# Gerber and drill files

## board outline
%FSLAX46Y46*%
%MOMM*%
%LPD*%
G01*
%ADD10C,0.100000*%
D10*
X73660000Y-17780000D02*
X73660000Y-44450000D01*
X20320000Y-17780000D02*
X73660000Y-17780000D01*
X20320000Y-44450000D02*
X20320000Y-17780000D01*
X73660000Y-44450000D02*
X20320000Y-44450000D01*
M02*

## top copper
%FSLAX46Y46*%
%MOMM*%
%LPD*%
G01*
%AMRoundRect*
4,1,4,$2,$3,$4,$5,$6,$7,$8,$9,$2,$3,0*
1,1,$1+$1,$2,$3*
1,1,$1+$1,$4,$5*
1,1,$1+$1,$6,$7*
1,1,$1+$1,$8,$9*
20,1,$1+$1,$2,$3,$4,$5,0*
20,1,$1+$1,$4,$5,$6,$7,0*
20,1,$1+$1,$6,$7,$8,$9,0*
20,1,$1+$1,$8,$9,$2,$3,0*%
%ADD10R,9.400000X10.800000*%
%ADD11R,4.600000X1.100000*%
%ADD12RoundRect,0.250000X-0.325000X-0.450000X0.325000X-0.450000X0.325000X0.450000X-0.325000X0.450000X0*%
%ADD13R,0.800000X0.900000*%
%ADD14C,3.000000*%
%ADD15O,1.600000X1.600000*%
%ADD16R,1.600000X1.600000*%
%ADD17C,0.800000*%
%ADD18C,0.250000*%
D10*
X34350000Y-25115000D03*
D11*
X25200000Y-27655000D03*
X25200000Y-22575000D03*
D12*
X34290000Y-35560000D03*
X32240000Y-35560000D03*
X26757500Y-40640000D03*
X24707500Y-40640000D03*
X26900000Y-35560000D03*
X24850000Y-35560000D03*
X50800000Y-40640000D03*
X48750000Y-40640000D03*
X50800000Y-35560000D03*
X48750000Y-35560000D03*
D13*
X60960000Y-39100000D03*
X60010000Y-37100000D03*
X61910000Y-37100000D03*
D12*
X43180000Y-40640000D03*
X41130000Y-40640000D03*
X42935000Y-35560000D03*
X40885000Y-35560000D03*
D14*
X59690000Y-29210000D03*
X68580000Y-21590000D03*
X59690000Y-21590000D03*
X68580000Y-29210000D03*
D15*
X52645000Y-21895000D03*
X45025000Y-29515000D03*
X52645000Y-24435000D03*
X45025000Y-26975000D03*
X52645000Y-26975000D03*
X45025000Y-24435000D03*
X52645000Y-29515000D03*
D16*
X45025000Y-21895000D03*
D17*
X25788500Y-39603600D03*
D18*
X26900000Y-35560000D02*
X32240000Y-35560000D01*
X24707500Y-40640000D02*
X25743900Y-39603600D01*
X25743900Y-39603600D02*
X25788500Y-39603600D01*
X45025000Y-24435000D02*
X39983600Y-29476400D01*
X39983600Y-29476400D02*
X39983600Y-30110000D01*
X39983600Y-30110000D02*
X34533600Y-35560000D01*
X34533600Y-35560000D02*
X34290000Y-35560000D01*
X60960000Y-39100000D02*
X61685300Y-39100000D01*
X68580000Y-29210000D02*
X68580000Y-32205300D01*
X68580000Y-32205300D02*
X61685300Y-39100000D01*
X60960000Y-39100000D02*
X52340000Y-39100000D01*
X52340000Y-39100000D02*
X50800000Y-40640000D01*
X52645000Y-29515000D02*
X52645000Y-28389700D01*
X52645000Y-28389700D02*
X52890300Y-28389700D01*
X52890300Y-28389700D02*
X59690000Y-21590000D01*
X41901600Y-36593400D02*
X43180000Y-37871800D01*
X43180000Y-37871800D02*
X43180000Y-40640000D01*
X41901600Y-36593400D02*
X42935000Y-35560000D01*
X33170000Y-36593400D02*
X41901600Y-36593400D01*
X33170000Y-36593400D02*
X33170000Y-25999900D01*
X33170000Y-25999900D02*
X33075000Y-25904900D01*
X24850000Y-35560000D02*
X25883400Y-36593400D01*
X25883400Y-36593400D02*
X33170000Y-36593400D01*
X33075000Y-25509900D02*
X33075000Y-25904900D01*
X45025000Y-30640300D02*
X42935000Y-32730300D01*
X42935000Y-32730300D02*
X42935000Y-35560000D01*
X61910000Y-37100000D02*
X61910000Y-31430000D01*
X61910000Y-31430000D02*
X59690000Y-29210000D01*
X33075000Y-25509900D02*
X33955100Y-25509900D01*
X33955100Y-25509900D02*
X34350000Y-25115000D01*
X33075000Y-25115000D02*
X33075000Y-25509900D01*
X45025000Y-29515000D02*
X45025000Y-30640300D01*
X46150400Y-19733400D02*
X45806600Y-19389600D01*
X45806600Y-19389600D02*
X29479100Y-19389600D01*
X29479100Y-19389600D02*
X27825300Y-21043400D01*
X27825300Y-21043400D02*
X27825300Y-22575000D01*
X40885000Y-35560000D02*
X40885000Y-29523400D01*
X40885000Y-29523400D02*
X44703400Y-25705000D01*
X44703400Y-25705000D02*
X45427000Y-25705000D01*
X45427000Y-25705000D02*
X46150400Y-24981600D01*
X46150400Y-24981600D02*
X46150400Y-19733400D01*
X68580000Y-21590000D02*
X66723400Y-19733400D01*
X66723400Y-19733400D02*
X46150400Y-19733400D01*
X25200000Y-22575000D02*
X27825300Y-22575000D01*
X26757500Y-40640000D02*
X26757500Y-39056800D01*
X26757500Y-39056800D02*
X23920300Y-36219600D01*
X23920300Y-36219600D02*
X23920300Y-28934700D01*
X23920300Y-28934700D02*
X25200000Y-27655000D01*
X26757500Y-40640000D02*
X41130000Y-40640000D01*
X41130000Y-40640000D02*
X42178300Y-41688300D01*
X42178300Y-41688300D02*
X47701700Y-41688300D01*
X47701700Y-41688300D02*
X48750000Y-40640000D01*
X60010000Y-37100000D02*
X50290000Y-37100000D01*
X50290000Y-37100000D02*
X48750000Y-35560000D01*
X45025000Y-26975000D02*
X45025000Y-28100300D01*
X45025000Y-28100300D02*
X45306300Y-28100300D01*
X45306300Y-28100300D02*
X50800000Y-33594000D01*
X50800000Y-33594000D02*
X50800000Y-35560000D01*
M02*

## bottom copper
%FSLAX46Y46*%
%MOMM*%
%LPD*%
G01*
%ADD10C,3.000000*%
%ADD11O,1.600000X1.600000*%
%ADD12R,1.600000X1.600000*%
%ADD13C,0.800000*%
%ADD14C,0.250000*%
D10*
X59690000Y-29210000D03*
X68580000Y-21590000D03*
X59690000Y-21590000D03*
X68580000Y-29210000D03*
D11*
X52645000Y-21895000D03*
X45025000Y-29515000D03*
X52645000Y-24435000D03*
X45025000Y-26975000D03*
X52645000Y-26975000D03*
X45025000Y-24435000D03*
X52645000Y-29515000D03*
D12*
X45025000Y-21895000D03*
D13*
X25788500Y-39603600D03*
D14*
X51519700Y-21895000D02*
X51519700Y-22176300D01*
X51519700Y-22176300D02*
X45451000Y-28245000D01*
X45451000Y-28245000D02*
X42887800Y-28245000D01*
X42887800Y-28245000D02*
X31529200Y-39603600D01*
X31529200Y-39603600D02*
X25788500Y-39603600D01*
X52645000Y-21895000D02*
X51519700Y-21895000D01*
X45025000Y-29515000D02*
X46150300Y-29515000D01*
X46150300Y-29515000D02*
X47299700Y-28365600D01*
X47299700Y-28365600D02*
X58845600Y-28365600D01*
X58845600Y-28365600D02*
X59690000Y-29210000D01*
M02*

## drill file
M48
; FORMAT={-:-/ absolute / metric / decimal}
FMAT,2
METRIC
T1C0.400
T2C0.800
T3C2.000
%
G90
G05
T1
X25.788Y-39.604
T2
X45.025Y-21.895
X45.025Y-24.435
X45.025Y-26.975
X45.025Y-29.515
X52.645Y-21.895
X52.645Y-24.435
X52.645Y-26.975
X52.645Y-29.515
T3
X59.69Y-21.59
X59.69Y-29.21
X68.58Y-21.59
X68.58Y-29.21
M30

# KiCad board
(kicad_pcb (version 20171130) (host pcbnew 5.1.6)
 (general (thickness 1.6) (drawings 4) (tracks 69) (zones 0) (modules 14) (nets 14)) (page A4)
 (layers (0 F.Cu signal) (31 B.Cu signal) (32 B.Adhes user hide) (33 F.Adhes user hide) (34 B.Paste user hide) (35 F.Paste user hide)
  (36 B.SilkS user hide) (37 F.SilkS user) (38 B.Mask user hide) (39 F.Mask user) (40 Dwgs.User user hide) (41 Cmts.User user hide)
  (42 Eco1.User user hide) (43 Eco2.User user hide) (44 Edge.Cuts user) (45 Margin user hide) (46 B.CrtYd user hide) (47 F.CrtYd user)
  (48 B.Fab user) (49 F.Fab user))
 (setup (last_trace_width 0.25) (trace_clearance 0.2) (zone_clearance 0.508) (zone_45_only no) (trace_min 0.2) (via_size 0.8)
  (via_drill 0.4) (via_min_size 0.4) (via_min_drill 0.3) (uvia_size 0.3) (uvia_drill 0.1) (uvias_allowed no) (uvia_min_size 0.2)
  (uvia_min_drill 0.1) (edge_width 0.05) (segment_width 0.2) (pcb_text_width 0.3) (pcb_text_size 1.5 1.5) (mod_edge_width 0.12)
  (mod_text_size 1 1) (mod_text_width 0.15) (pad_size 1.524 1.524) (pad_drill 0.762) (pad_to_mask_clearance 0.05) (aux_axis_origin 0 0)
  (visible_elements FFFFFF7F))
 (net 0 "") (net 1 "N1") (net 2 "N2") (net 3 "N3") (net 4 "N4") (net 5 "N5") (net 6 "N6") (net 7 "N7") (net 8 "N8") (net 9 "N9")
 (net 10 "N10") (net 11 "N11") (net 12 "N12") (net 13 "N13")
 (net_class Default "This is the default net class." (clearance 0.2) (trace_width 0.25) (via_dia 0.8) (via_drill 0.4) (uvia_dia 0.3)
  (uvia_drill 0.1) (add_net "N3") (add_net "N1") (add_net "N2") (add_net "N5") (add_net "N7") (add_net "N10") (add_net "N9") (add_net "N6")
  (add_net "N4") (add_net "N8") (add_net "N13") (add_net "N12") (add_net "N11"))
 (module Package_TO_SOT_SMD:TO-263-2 (layer F.Cu) (at 30.975 25.115)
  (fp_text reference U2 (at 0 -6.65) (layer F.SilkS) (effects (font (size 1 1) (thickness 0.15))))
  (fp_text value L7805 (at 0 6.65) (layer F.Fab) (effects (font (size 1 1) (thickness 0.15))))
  (pad "" smd rect (at 0.95 2.775) (size 4.55 5.25) (layers F.Paste))
  (pad "" smd rect (at 5.8 -2.775) (size 4.55 5.25) (layers F.Paste))
  (pad "" smd rect (at 0.95 -2.775) (size 4.55 5.25) (layers F.Paste))
  (pad "" smd rect (at 5.8 2.775) (size 4.55 5.25) (layers F.Paste))
  (pad 2 smd rect (at 3.375 0) (size 9.4 10.8) (layers F.Cu F.Mask) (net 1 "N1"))
  (pad 3 smd rect (at -5.775 2.54) (size 4.6 1.1) (layers F.Cu F.Paste F.Mask) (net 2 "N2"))
  (pad 1 smd rect (at -5.775 -2.54) (size 4.6 1.1) (layers F.Cu F.Paste F.Mask) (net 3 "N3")))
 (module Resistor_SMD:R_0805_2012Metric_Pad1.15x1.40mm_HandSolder (layer F.Cu) (at 33.265 35.56)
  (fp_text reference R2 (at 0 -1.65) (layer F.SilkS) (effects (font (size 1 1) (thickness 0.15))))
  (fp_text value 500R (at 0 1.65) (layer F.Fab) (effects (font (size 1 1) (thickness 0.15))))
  (pad 2 smd roundrect (at 1.025 0) (size 1.15 1.4) (layers F.Cu F.Paste F.Mask) (roundrect_rratio 0.217391) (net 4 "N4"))
  (pad 1 smd roundrect (at -1.025 0) (size 1.15 1.4) (layers F.Cu F.Paste F.Mask) (roundrect_rratio 0.217391) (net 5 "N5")))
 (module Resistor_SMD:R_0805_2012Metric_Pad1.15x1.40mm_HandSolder (layer F.Cu) (at 25.7325 40.64)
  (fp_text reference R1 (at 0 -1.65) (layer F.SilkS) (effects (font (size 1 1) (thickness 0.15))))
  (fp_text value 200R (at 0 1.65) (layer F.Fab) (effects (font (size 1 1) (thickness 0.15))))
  (pad 2 smd roundrect (at 1.025 0) (size 1.15 1.4) (layers F.Cu F.Paste F.Mask) (roundrect_rratio 0.217391) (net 2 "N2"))
  (pad 1 smd roundrect (at -1.025 0) (size 1.15 1.4) (layers F.Cu F.Paste F.Mask) (roundrect_rratio 0.217391) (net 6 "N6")))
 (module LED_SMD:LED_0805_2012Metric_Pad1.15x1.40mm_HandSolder (layer F.Cu) (at 25.875 35.56)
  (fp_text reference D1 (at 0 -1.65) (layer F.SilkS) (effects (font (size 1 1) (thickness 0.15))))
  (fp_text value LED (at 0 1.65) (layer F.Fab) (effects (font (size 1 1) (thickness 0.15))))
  (pad 2 smd roundrect (at 1.025 0) (size 1.15 1.4) (layers F.Cu F.Paste F.Mask) (roundrect_rratio 0.217391) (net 5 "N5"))
  (pad 1 smd roundrect (at -1.025 0) (size 1.15 1.4) (layers F.Cu F.Paste F.Mask) (roundrect_rratio 0.217391) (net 1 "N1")))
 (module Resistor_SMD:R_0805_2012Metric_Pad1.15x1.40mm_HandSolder (layer F.Cu) (at 49.775 40.64)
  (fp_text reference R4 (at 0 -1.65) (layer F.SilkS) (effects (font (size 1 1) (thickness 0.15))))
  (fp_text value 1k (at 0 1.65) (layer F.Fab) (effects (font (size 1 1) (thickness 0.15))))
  (pad 2 smd roundrect (at 1.025 0) (size 1.15 1.4) (layers F.Cu F.Paste F.Mask) (roundrect_rratio 0.217391) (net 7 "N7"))
  (pad 1 smd roundrect (at -1.025 0) (size 1.15 1.4) (layers F.Cu F.Paste F.Mask) (roundrect_rratio 0.217391) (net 2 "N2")))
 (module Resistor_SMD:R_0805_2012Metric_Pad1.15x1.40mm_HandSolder (layer F.Cu) (at 49.775 35.56)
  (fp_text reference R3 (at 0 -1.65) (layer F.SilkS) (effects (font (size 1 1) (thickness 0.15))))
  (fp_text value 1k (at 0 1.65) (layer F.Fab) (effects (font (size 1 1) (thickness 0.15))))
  (pad 2 smd roundrect (at 1.025 0) (size 1.15 1.4) (layers F.Cu F.Paste F.Mask) (roundrect_rratio 0.217391) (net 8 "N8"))
  (pad 1 smd roundrect (at -1.025 0) (size 1.15 1.4) (layers F.Cu F.Paste F.Mask) (roundrect_rratio 0.217391) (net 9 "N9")))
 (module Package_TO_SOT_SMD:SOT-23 (layer F.Cu) (at 60.96 38.1 270)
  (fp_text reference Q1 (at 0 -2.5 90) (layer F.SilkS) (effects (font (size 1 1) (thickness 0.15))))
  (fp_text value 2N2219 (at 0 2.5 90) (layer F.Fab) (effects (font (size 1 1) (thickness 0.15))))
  (pad 3 smd rect (at 1 0 270) (size 0.9 0.8) (layers F.Cu F.Paste F.Mask) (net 7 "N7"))
  (pad 2 smd rect (at -1 0.95 270) (size 0.9 0.8) (layers F.Cu F.Paste F.Mask) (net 9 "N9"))
  (pad 1 smd rect (at -1 -0.95 270) (size 0.9 0.8) (layers F.Cu F.Paste F.Mask) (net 1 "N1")))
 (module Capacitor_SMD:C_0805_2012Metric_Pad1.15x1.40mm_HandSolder (layer F.Cu) (at 42.155 40.64)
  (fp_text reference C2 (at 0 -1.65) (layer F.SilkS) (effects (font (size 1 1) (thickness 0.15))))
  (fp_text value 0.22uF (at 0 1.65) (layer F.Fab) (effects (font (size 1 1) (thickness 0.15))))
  (pad 2 smd roundrect (at 1.025 0) (size 1.15 1.4) (layers F.Cu F.Paste F.Mask) (roundrect_rratio 0.217391) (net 1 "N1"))
  (pad 1 smd roundrect (at -1.025 0) (size 1.15 1.4) (layers F.Cu F.Paste F.Mask) (roundrect_rratio 0.217391) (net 2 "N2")))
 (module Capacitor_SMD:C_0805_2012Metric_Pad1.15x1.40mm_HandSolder (layer F.Cu) (at 41.91 35.56)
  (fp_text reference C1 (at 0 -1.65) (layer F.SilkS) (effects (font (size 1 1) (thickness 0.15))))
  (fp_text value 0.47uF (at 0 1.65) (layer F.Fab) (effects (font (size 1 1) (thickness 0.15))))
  (pad 2 smd roundrect (at 1.025 0) (size 1.15 1.4) (layers F.Cu F.Paste F.Mask) (roundrect_rratio 0.217391) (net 1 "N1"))
  (pad 1 smd roundrect (at -1.025 0) (size 1.15 1.4) (layers F.Cu F.Paste F.Mask) (roundrect_rratio 0.217391) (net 3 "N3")))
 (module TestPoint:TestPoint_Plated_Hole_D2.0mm (layer F.Cu) (at 59.69 29.21)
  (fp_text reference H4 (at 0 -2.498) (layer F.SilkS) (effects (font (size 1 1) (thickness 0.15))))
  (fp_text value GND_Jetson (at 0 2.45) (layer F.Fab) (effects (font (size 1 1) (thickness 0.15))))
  (pad 1 thru_hole circle (at 0 0) (size 3 3) (drill 2) (layers *.Cu *.Mask) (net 1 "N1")))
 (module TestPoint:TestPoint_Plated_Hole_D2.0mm (layer F.Cu) (at 68.58 21.59)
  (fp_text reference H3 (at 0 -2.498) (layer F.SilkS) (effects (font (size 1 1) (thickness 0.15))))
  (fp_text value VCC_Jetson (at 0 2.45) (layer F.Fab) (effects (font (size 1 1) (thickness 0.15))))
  (pad 1 thru_hole circle (at 0 0) (size 3 3) (drill 2) (layers *.Cu *.Mask) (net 3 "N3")))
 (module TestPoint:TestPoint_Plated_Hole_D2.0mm (layer F.Cu) (at 59.69 21.59)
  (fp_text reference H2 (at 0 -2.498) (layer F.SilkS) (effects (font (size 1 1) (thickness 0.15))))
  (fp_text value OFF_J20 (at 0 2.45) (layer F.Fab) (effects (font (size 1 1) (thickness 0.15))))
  (pad 1 thru_hole circle (at 0 0) (size 3 3) (drill 2) (layers *.Cu *.Mask) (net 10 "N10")))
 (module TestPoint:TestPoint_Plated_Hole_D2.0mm (layer F.Cu) (at 68.58 29.21)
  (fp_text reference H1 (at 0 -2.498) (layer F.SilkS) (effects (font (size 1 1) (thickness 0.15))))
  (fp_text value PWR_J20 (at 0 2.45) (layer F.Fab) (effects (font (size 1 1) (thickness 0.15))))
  (pad 1 thru_hole circle (at 0 0) (size 3 3) (drill 2) (layers *.Cu *.Mask) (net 7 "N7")))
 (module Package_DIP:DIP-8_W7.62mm (layer F.Cu) (at 45.025 21.895)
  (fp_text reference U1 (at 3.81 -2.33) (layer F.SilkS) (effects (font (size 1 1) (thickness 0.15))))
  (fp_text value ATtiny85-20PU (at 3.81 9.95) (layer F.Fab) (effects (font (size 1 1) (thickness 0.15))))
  (pad 8 thru_hole oval (at 7.62 0) (size 1.6 1.6) (drill 0.8) (layers *.Cu *.Mask) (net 6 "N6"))
  (pad 4 thru_hole oval (at 0 7.62) (size 1.6 1.6) (drill 0.8) (layers *.Cu *.Mask) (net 1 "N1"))
  (pad 7 thru_hole oval (at 7.62 2.54) (size 1.6 1.6) (drill 0.8) (layers *.Cu *.Mask) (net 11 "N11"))
  (pad 3 thru_hole oval (at 0 5.08) (size 1.6 1.6) (drill 0.8) (layers *.Cu *.Mask) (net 8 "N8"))
  (pad 6 thru_hole oval (at 7.62 5.08) (size 1.6 1.6) (drill 0.8) (layers *.Cu *.Mask) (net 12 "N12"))
  (pad 2 thru_hole oval (at 0 2.54) (size 1.6 1.6) (drill 0.8) (layers *.Cu *.Mask) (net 4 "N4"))
  (pad 5 thru_hole oval (at 7.62 7.62) (size 1.6 1.6) (drill 0.8) (layers *.Cu *.Mask) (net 10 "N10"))
  (pad 1 thru_hole rect (at 0 0) (size 1.6 1.6) (drill 0.8) (layers *.Cu *.Mask) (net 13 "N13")))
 (gr_line (start 73.66 17.78) (end 73.66 44.45) (layer Edge.Cuts) (width 0.1))
 (gr_line (start 20.32 17.78) (end 73.66 17.78) (layer Edge.Cuts) (width 0.1))
 (gr_line (start 20.32 44.45) (end 20.32 17.78) (layer Edge.Cuts) (width 0.1))
 (gr_line (start 73.66 44.45) (end 20.32 44.45) (layer Edge.Cuts) (width 0.1))
 (segment (start 26.9 35.56) (end 32.24 35.56) (width 0.25) (layer F.Cu) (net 5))
 (segment (start 24.7075 40.64) (end 25.7439 39.6036) (width 0.25) (layer F.Cu) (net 6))
 (segment (start 25.7439 39.6036) (end 25.7885 39.6036) (width 0.25) (layer F.Cu) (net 6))
 (segment (start 51.5197 21.895) (end 51.5197 22.1763) (width 0.25) (layer B.Cu) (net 6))
 (segment (start 51.5197 22.1763) (end 45.451 28.245) (width 0.25) (layer B.Cu) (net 6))
 (segment (start 45.451 28.245) (end 42.8878 28.245) (width 0.25) (layer B.Cu) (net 6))
 (segment (start 42.8878 28.245) (end 31.5292 39.6036) (width 0.25) (layer B.Cu) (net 6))
 (segment (start 31.5292 39.6036) (end 25.7885 39.6036) (width 0.25) (layer B.Cu) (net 6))
 (segment (start 52.645 21.895) (end 51.5197 21.895) (width 0.25) (layer B.Cu) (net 6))
 (via (at 25.7885 39.6036) (size 0.8) (layers F.Cu B.Cu) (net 6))
 (segment (start 45.025 24.435) (end 39.9836 29.4764) (width 0.25) (layer F.Cu) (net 4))
 (segment (start 39.9836 29.4764) (end 39.9836 30.11) (width 0.25) (layer F.Cu) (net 4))
 (segment (start 39.9836 30.11) (end 34.5336 35.56) (width 0.25) (layer F.Cu) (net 4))
 (segment (start 34.5336 35.56) (end 34.29 35.56) (width 0.25) (layer F.Cu) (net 4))
 (segment (start 60.96 39.1) (end 61.6853 39.1) (width 0.25) (layer F.Cu) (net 7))
 (segment (start 68.58 29.21) (end 68.58 32.2053) (width 0.25) (layer F.Cu) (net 7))
 (segment (start 68.58 32.2053) (end 61.6853 39.1) (width 0.25) (layer F.Cu) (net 7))
 (segment (start 60.96 39.1) (end 52.34 39.1) (width 0.25) (layer F.Cu) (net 7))
 (segment (start 52.34 39.1) (end 50.8 40.64) (width 0.25) (layer F.Cu) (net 7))
 (segment (start 52.645 29.515) (end 52.645 28.3897) (width 0.25) (layer F.Cu) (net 10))
 (segment (start 52.645 28.3897) (end 52.8903 28.3897) (width 0.25) (layer F.Cu) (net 10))
 (segment (start 52.8903 28.3897) (end 59.69 21.59) (width 0.25) (layer F.Cu) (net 10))
 (segment (start 41.9016 36.5934) (end 43.18 37.8718) (width 0.25) (layer F.Cu) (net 1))
 (segment (start 43.18 37.8718) (end 43.18 40.64) (width 0.25) (layer F.Cu) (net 1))
 (segment (start 41.9016 36.5934) (end 42.935 35.56) (width 0.25) (layer F.Cu) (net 1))
 (segment (start 33.17 36.5934) (end 41.9016 36.5934) (width 0.25) (layer F.Cu) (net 1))
 (segment (start 33.17 36.5934) (end 33.17 25.9999) (width 0.25) (layer F.Cu) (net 1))
 (segment (start 33.17 25.9999) (end 33.075 25.9049) (width 0.25) (layer F.Cu) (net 1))
 (segment (start 24.85 35.56) (end 25.8834 36.5934) (width 0.25) (layer F.Cu) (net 1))
 (segment (start 25.8834 36.5934) (end 33.17 36.5934) (width 0.25) (layer F.Cu) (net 1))
 (segment (start 33.075 25.5099) (end 33.075 25.9049) (width 0.25) (layer F.Cu) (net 1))
 (segment (start 45.025 29.515) (end 46.1503 29.515) (width 0.25) (layer B.Cu) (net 1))
 (segment (start 46.1503 29.515) (end 47.2997 28.3656) (width 0.25) (layer B.Cu) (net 1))
 (segment (start 47.2997 28.3656) (end 58.8456 28.3656) (width 0.25) (layer B.Cu) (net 1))
 (segment (start 58.8456 28.3656) (end 59.69 29.21) (width 0.25) (layer B.Cu) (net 1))
 (segment (start 45.025 30.6403) (end 42.935 32.7303) (width 0.25) (layer F.Cu) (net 1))
 (segment (start 42.935 32.7303) (end 42.935 35.56) (width 0.25) (layer F.Cu) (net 1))
 (segment (start 61.91 37.1) (end 61.91 31.43) (width 0.25) (layer F.Cu) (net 1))
 (segment (start 61.91 31.43) (end 59.69 29.21) (width 0.25) (layer F.Cu) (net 1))
 (segment (start 33.075 25.5099) (end 33.9551 25.5099) (width 0.25) (layer F.Cu) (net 1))
 (segment (start 33.9551 25.5099) (end 34.35 25.115) (width 0.25) (layer F.Cu) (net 1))
 (segment (start 33.075 25.115) (end 33.075 25.5099) (width 0.25) (layer F.Cu) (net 1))
 (segment (start 45.025 29.515) (end 45.025 30.6403) (width 0.25) (layer F.Cu) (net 1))
 (segment (start 46.1504 19.7334) (end 45.8066 19.3896) (width 0.25) (layer F.Cu) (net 3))
 (segment (start 45.8066 19.3896) (end 29.4791 19.3896) (width 0.25) (layer F.Cu) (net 3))
 (segment (start 29.4791 19.3896) (end 27.8253 21.0434) (width 0.25) (layer F.Cu) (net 3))
 (segment (start 27.8253 21.0434) (end 27.8253 22.575) (width 0.25) (layer F.Cu) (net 3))
 (segment (start 40.885 35.56) (end 40.885 29.5234) (width 0.25) (layer F.Cu) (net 3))
 (segment (start 40.885 29.5234) (end 44.7034 25.705) (width 0.25) (layer F.Cu) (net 3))
 (segment (start 44.7034 25.705) (end 45.427 25.705) (width 0.25) (layer F.Cu) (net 3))
 (segment (start 45.427 25.705) (end 46.1504 24.9816) (width 0.25) (layer F.Cu) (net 3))
 (segment (start 46.1504 24.9816) (end 46.1504 19.7334) (width 0.25) (layer F.Cu) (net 3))
 (segment (start 68.58 21.59) (end 66.7234 19.7334) (width 0.25) (layer F.Cu) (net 3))
 (segment (start 66.7234 19.7334) (end 46.1504 19.7334) (width 0.25) (layer F.Cu) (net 3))
 (segment (start 25.2 22.575) (end 27.8253 22.575) (width 0.25) (layer F.Cu) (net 3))
 (segment (start 26.7575 40.64) (end 26.7575 39.0568) (width 0.25) (layer F.Cu) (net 2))
 (segment (start 26.7575 39.0568) (end 23.9203 36.2196) (width 0.25) (layer F.Cu) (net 2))
 (segment (start 23.9203 36.2196) (end 23.9203 28.9347) (width 0.25) (layer F.Cu) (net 2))
 (segment (start 23.9203 28.9347) (end 25.2 27.655) (width 0.25) (layer F.Cu) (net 2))
 (segment (start 26.7575 40.64) (end 41.13 40.64) (width 0.25) (layer F.Cu) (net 2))
 (segment (start 41.13 40.64) (end 42.1783 41.6883) (width 0.25) (layer F.Cu) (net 2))
 (segment (start 42.1783 41.6883) (end 47.7017 41.6883) (width 0.25) (layer F.Cu) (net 2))
 (segment (start 47.7017 41.6883) (end 48.75 40.64) (width 0.25) (layer F.Cu) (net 2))
 (segment (start 60.01 37.1) (end 50.29 37.1) (width 0.25) (layer F.Cu) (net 9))
 (segment (start 50.29 37.1) (end 48.75 35.56) (width 0.25) (layer F.Cu) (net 9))
 (segment (start 45.025 26.975) (end 45.025 28.1003) (width 0.25) (layer F.Cu) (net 8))
 (segment (start 45.025 28.1003) (end 45.3063 28.1003) (width 0.25) (layer F.Cu) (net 8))
 (segment (start 45.3063 28.1003) (end 50.8 33.594) (width 0.25) (layer F.Cu) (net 8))
 (segment (start 50.8 33.594) (end 50.8 35.56) (width 0.25) (layer F.Cu) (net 8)))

